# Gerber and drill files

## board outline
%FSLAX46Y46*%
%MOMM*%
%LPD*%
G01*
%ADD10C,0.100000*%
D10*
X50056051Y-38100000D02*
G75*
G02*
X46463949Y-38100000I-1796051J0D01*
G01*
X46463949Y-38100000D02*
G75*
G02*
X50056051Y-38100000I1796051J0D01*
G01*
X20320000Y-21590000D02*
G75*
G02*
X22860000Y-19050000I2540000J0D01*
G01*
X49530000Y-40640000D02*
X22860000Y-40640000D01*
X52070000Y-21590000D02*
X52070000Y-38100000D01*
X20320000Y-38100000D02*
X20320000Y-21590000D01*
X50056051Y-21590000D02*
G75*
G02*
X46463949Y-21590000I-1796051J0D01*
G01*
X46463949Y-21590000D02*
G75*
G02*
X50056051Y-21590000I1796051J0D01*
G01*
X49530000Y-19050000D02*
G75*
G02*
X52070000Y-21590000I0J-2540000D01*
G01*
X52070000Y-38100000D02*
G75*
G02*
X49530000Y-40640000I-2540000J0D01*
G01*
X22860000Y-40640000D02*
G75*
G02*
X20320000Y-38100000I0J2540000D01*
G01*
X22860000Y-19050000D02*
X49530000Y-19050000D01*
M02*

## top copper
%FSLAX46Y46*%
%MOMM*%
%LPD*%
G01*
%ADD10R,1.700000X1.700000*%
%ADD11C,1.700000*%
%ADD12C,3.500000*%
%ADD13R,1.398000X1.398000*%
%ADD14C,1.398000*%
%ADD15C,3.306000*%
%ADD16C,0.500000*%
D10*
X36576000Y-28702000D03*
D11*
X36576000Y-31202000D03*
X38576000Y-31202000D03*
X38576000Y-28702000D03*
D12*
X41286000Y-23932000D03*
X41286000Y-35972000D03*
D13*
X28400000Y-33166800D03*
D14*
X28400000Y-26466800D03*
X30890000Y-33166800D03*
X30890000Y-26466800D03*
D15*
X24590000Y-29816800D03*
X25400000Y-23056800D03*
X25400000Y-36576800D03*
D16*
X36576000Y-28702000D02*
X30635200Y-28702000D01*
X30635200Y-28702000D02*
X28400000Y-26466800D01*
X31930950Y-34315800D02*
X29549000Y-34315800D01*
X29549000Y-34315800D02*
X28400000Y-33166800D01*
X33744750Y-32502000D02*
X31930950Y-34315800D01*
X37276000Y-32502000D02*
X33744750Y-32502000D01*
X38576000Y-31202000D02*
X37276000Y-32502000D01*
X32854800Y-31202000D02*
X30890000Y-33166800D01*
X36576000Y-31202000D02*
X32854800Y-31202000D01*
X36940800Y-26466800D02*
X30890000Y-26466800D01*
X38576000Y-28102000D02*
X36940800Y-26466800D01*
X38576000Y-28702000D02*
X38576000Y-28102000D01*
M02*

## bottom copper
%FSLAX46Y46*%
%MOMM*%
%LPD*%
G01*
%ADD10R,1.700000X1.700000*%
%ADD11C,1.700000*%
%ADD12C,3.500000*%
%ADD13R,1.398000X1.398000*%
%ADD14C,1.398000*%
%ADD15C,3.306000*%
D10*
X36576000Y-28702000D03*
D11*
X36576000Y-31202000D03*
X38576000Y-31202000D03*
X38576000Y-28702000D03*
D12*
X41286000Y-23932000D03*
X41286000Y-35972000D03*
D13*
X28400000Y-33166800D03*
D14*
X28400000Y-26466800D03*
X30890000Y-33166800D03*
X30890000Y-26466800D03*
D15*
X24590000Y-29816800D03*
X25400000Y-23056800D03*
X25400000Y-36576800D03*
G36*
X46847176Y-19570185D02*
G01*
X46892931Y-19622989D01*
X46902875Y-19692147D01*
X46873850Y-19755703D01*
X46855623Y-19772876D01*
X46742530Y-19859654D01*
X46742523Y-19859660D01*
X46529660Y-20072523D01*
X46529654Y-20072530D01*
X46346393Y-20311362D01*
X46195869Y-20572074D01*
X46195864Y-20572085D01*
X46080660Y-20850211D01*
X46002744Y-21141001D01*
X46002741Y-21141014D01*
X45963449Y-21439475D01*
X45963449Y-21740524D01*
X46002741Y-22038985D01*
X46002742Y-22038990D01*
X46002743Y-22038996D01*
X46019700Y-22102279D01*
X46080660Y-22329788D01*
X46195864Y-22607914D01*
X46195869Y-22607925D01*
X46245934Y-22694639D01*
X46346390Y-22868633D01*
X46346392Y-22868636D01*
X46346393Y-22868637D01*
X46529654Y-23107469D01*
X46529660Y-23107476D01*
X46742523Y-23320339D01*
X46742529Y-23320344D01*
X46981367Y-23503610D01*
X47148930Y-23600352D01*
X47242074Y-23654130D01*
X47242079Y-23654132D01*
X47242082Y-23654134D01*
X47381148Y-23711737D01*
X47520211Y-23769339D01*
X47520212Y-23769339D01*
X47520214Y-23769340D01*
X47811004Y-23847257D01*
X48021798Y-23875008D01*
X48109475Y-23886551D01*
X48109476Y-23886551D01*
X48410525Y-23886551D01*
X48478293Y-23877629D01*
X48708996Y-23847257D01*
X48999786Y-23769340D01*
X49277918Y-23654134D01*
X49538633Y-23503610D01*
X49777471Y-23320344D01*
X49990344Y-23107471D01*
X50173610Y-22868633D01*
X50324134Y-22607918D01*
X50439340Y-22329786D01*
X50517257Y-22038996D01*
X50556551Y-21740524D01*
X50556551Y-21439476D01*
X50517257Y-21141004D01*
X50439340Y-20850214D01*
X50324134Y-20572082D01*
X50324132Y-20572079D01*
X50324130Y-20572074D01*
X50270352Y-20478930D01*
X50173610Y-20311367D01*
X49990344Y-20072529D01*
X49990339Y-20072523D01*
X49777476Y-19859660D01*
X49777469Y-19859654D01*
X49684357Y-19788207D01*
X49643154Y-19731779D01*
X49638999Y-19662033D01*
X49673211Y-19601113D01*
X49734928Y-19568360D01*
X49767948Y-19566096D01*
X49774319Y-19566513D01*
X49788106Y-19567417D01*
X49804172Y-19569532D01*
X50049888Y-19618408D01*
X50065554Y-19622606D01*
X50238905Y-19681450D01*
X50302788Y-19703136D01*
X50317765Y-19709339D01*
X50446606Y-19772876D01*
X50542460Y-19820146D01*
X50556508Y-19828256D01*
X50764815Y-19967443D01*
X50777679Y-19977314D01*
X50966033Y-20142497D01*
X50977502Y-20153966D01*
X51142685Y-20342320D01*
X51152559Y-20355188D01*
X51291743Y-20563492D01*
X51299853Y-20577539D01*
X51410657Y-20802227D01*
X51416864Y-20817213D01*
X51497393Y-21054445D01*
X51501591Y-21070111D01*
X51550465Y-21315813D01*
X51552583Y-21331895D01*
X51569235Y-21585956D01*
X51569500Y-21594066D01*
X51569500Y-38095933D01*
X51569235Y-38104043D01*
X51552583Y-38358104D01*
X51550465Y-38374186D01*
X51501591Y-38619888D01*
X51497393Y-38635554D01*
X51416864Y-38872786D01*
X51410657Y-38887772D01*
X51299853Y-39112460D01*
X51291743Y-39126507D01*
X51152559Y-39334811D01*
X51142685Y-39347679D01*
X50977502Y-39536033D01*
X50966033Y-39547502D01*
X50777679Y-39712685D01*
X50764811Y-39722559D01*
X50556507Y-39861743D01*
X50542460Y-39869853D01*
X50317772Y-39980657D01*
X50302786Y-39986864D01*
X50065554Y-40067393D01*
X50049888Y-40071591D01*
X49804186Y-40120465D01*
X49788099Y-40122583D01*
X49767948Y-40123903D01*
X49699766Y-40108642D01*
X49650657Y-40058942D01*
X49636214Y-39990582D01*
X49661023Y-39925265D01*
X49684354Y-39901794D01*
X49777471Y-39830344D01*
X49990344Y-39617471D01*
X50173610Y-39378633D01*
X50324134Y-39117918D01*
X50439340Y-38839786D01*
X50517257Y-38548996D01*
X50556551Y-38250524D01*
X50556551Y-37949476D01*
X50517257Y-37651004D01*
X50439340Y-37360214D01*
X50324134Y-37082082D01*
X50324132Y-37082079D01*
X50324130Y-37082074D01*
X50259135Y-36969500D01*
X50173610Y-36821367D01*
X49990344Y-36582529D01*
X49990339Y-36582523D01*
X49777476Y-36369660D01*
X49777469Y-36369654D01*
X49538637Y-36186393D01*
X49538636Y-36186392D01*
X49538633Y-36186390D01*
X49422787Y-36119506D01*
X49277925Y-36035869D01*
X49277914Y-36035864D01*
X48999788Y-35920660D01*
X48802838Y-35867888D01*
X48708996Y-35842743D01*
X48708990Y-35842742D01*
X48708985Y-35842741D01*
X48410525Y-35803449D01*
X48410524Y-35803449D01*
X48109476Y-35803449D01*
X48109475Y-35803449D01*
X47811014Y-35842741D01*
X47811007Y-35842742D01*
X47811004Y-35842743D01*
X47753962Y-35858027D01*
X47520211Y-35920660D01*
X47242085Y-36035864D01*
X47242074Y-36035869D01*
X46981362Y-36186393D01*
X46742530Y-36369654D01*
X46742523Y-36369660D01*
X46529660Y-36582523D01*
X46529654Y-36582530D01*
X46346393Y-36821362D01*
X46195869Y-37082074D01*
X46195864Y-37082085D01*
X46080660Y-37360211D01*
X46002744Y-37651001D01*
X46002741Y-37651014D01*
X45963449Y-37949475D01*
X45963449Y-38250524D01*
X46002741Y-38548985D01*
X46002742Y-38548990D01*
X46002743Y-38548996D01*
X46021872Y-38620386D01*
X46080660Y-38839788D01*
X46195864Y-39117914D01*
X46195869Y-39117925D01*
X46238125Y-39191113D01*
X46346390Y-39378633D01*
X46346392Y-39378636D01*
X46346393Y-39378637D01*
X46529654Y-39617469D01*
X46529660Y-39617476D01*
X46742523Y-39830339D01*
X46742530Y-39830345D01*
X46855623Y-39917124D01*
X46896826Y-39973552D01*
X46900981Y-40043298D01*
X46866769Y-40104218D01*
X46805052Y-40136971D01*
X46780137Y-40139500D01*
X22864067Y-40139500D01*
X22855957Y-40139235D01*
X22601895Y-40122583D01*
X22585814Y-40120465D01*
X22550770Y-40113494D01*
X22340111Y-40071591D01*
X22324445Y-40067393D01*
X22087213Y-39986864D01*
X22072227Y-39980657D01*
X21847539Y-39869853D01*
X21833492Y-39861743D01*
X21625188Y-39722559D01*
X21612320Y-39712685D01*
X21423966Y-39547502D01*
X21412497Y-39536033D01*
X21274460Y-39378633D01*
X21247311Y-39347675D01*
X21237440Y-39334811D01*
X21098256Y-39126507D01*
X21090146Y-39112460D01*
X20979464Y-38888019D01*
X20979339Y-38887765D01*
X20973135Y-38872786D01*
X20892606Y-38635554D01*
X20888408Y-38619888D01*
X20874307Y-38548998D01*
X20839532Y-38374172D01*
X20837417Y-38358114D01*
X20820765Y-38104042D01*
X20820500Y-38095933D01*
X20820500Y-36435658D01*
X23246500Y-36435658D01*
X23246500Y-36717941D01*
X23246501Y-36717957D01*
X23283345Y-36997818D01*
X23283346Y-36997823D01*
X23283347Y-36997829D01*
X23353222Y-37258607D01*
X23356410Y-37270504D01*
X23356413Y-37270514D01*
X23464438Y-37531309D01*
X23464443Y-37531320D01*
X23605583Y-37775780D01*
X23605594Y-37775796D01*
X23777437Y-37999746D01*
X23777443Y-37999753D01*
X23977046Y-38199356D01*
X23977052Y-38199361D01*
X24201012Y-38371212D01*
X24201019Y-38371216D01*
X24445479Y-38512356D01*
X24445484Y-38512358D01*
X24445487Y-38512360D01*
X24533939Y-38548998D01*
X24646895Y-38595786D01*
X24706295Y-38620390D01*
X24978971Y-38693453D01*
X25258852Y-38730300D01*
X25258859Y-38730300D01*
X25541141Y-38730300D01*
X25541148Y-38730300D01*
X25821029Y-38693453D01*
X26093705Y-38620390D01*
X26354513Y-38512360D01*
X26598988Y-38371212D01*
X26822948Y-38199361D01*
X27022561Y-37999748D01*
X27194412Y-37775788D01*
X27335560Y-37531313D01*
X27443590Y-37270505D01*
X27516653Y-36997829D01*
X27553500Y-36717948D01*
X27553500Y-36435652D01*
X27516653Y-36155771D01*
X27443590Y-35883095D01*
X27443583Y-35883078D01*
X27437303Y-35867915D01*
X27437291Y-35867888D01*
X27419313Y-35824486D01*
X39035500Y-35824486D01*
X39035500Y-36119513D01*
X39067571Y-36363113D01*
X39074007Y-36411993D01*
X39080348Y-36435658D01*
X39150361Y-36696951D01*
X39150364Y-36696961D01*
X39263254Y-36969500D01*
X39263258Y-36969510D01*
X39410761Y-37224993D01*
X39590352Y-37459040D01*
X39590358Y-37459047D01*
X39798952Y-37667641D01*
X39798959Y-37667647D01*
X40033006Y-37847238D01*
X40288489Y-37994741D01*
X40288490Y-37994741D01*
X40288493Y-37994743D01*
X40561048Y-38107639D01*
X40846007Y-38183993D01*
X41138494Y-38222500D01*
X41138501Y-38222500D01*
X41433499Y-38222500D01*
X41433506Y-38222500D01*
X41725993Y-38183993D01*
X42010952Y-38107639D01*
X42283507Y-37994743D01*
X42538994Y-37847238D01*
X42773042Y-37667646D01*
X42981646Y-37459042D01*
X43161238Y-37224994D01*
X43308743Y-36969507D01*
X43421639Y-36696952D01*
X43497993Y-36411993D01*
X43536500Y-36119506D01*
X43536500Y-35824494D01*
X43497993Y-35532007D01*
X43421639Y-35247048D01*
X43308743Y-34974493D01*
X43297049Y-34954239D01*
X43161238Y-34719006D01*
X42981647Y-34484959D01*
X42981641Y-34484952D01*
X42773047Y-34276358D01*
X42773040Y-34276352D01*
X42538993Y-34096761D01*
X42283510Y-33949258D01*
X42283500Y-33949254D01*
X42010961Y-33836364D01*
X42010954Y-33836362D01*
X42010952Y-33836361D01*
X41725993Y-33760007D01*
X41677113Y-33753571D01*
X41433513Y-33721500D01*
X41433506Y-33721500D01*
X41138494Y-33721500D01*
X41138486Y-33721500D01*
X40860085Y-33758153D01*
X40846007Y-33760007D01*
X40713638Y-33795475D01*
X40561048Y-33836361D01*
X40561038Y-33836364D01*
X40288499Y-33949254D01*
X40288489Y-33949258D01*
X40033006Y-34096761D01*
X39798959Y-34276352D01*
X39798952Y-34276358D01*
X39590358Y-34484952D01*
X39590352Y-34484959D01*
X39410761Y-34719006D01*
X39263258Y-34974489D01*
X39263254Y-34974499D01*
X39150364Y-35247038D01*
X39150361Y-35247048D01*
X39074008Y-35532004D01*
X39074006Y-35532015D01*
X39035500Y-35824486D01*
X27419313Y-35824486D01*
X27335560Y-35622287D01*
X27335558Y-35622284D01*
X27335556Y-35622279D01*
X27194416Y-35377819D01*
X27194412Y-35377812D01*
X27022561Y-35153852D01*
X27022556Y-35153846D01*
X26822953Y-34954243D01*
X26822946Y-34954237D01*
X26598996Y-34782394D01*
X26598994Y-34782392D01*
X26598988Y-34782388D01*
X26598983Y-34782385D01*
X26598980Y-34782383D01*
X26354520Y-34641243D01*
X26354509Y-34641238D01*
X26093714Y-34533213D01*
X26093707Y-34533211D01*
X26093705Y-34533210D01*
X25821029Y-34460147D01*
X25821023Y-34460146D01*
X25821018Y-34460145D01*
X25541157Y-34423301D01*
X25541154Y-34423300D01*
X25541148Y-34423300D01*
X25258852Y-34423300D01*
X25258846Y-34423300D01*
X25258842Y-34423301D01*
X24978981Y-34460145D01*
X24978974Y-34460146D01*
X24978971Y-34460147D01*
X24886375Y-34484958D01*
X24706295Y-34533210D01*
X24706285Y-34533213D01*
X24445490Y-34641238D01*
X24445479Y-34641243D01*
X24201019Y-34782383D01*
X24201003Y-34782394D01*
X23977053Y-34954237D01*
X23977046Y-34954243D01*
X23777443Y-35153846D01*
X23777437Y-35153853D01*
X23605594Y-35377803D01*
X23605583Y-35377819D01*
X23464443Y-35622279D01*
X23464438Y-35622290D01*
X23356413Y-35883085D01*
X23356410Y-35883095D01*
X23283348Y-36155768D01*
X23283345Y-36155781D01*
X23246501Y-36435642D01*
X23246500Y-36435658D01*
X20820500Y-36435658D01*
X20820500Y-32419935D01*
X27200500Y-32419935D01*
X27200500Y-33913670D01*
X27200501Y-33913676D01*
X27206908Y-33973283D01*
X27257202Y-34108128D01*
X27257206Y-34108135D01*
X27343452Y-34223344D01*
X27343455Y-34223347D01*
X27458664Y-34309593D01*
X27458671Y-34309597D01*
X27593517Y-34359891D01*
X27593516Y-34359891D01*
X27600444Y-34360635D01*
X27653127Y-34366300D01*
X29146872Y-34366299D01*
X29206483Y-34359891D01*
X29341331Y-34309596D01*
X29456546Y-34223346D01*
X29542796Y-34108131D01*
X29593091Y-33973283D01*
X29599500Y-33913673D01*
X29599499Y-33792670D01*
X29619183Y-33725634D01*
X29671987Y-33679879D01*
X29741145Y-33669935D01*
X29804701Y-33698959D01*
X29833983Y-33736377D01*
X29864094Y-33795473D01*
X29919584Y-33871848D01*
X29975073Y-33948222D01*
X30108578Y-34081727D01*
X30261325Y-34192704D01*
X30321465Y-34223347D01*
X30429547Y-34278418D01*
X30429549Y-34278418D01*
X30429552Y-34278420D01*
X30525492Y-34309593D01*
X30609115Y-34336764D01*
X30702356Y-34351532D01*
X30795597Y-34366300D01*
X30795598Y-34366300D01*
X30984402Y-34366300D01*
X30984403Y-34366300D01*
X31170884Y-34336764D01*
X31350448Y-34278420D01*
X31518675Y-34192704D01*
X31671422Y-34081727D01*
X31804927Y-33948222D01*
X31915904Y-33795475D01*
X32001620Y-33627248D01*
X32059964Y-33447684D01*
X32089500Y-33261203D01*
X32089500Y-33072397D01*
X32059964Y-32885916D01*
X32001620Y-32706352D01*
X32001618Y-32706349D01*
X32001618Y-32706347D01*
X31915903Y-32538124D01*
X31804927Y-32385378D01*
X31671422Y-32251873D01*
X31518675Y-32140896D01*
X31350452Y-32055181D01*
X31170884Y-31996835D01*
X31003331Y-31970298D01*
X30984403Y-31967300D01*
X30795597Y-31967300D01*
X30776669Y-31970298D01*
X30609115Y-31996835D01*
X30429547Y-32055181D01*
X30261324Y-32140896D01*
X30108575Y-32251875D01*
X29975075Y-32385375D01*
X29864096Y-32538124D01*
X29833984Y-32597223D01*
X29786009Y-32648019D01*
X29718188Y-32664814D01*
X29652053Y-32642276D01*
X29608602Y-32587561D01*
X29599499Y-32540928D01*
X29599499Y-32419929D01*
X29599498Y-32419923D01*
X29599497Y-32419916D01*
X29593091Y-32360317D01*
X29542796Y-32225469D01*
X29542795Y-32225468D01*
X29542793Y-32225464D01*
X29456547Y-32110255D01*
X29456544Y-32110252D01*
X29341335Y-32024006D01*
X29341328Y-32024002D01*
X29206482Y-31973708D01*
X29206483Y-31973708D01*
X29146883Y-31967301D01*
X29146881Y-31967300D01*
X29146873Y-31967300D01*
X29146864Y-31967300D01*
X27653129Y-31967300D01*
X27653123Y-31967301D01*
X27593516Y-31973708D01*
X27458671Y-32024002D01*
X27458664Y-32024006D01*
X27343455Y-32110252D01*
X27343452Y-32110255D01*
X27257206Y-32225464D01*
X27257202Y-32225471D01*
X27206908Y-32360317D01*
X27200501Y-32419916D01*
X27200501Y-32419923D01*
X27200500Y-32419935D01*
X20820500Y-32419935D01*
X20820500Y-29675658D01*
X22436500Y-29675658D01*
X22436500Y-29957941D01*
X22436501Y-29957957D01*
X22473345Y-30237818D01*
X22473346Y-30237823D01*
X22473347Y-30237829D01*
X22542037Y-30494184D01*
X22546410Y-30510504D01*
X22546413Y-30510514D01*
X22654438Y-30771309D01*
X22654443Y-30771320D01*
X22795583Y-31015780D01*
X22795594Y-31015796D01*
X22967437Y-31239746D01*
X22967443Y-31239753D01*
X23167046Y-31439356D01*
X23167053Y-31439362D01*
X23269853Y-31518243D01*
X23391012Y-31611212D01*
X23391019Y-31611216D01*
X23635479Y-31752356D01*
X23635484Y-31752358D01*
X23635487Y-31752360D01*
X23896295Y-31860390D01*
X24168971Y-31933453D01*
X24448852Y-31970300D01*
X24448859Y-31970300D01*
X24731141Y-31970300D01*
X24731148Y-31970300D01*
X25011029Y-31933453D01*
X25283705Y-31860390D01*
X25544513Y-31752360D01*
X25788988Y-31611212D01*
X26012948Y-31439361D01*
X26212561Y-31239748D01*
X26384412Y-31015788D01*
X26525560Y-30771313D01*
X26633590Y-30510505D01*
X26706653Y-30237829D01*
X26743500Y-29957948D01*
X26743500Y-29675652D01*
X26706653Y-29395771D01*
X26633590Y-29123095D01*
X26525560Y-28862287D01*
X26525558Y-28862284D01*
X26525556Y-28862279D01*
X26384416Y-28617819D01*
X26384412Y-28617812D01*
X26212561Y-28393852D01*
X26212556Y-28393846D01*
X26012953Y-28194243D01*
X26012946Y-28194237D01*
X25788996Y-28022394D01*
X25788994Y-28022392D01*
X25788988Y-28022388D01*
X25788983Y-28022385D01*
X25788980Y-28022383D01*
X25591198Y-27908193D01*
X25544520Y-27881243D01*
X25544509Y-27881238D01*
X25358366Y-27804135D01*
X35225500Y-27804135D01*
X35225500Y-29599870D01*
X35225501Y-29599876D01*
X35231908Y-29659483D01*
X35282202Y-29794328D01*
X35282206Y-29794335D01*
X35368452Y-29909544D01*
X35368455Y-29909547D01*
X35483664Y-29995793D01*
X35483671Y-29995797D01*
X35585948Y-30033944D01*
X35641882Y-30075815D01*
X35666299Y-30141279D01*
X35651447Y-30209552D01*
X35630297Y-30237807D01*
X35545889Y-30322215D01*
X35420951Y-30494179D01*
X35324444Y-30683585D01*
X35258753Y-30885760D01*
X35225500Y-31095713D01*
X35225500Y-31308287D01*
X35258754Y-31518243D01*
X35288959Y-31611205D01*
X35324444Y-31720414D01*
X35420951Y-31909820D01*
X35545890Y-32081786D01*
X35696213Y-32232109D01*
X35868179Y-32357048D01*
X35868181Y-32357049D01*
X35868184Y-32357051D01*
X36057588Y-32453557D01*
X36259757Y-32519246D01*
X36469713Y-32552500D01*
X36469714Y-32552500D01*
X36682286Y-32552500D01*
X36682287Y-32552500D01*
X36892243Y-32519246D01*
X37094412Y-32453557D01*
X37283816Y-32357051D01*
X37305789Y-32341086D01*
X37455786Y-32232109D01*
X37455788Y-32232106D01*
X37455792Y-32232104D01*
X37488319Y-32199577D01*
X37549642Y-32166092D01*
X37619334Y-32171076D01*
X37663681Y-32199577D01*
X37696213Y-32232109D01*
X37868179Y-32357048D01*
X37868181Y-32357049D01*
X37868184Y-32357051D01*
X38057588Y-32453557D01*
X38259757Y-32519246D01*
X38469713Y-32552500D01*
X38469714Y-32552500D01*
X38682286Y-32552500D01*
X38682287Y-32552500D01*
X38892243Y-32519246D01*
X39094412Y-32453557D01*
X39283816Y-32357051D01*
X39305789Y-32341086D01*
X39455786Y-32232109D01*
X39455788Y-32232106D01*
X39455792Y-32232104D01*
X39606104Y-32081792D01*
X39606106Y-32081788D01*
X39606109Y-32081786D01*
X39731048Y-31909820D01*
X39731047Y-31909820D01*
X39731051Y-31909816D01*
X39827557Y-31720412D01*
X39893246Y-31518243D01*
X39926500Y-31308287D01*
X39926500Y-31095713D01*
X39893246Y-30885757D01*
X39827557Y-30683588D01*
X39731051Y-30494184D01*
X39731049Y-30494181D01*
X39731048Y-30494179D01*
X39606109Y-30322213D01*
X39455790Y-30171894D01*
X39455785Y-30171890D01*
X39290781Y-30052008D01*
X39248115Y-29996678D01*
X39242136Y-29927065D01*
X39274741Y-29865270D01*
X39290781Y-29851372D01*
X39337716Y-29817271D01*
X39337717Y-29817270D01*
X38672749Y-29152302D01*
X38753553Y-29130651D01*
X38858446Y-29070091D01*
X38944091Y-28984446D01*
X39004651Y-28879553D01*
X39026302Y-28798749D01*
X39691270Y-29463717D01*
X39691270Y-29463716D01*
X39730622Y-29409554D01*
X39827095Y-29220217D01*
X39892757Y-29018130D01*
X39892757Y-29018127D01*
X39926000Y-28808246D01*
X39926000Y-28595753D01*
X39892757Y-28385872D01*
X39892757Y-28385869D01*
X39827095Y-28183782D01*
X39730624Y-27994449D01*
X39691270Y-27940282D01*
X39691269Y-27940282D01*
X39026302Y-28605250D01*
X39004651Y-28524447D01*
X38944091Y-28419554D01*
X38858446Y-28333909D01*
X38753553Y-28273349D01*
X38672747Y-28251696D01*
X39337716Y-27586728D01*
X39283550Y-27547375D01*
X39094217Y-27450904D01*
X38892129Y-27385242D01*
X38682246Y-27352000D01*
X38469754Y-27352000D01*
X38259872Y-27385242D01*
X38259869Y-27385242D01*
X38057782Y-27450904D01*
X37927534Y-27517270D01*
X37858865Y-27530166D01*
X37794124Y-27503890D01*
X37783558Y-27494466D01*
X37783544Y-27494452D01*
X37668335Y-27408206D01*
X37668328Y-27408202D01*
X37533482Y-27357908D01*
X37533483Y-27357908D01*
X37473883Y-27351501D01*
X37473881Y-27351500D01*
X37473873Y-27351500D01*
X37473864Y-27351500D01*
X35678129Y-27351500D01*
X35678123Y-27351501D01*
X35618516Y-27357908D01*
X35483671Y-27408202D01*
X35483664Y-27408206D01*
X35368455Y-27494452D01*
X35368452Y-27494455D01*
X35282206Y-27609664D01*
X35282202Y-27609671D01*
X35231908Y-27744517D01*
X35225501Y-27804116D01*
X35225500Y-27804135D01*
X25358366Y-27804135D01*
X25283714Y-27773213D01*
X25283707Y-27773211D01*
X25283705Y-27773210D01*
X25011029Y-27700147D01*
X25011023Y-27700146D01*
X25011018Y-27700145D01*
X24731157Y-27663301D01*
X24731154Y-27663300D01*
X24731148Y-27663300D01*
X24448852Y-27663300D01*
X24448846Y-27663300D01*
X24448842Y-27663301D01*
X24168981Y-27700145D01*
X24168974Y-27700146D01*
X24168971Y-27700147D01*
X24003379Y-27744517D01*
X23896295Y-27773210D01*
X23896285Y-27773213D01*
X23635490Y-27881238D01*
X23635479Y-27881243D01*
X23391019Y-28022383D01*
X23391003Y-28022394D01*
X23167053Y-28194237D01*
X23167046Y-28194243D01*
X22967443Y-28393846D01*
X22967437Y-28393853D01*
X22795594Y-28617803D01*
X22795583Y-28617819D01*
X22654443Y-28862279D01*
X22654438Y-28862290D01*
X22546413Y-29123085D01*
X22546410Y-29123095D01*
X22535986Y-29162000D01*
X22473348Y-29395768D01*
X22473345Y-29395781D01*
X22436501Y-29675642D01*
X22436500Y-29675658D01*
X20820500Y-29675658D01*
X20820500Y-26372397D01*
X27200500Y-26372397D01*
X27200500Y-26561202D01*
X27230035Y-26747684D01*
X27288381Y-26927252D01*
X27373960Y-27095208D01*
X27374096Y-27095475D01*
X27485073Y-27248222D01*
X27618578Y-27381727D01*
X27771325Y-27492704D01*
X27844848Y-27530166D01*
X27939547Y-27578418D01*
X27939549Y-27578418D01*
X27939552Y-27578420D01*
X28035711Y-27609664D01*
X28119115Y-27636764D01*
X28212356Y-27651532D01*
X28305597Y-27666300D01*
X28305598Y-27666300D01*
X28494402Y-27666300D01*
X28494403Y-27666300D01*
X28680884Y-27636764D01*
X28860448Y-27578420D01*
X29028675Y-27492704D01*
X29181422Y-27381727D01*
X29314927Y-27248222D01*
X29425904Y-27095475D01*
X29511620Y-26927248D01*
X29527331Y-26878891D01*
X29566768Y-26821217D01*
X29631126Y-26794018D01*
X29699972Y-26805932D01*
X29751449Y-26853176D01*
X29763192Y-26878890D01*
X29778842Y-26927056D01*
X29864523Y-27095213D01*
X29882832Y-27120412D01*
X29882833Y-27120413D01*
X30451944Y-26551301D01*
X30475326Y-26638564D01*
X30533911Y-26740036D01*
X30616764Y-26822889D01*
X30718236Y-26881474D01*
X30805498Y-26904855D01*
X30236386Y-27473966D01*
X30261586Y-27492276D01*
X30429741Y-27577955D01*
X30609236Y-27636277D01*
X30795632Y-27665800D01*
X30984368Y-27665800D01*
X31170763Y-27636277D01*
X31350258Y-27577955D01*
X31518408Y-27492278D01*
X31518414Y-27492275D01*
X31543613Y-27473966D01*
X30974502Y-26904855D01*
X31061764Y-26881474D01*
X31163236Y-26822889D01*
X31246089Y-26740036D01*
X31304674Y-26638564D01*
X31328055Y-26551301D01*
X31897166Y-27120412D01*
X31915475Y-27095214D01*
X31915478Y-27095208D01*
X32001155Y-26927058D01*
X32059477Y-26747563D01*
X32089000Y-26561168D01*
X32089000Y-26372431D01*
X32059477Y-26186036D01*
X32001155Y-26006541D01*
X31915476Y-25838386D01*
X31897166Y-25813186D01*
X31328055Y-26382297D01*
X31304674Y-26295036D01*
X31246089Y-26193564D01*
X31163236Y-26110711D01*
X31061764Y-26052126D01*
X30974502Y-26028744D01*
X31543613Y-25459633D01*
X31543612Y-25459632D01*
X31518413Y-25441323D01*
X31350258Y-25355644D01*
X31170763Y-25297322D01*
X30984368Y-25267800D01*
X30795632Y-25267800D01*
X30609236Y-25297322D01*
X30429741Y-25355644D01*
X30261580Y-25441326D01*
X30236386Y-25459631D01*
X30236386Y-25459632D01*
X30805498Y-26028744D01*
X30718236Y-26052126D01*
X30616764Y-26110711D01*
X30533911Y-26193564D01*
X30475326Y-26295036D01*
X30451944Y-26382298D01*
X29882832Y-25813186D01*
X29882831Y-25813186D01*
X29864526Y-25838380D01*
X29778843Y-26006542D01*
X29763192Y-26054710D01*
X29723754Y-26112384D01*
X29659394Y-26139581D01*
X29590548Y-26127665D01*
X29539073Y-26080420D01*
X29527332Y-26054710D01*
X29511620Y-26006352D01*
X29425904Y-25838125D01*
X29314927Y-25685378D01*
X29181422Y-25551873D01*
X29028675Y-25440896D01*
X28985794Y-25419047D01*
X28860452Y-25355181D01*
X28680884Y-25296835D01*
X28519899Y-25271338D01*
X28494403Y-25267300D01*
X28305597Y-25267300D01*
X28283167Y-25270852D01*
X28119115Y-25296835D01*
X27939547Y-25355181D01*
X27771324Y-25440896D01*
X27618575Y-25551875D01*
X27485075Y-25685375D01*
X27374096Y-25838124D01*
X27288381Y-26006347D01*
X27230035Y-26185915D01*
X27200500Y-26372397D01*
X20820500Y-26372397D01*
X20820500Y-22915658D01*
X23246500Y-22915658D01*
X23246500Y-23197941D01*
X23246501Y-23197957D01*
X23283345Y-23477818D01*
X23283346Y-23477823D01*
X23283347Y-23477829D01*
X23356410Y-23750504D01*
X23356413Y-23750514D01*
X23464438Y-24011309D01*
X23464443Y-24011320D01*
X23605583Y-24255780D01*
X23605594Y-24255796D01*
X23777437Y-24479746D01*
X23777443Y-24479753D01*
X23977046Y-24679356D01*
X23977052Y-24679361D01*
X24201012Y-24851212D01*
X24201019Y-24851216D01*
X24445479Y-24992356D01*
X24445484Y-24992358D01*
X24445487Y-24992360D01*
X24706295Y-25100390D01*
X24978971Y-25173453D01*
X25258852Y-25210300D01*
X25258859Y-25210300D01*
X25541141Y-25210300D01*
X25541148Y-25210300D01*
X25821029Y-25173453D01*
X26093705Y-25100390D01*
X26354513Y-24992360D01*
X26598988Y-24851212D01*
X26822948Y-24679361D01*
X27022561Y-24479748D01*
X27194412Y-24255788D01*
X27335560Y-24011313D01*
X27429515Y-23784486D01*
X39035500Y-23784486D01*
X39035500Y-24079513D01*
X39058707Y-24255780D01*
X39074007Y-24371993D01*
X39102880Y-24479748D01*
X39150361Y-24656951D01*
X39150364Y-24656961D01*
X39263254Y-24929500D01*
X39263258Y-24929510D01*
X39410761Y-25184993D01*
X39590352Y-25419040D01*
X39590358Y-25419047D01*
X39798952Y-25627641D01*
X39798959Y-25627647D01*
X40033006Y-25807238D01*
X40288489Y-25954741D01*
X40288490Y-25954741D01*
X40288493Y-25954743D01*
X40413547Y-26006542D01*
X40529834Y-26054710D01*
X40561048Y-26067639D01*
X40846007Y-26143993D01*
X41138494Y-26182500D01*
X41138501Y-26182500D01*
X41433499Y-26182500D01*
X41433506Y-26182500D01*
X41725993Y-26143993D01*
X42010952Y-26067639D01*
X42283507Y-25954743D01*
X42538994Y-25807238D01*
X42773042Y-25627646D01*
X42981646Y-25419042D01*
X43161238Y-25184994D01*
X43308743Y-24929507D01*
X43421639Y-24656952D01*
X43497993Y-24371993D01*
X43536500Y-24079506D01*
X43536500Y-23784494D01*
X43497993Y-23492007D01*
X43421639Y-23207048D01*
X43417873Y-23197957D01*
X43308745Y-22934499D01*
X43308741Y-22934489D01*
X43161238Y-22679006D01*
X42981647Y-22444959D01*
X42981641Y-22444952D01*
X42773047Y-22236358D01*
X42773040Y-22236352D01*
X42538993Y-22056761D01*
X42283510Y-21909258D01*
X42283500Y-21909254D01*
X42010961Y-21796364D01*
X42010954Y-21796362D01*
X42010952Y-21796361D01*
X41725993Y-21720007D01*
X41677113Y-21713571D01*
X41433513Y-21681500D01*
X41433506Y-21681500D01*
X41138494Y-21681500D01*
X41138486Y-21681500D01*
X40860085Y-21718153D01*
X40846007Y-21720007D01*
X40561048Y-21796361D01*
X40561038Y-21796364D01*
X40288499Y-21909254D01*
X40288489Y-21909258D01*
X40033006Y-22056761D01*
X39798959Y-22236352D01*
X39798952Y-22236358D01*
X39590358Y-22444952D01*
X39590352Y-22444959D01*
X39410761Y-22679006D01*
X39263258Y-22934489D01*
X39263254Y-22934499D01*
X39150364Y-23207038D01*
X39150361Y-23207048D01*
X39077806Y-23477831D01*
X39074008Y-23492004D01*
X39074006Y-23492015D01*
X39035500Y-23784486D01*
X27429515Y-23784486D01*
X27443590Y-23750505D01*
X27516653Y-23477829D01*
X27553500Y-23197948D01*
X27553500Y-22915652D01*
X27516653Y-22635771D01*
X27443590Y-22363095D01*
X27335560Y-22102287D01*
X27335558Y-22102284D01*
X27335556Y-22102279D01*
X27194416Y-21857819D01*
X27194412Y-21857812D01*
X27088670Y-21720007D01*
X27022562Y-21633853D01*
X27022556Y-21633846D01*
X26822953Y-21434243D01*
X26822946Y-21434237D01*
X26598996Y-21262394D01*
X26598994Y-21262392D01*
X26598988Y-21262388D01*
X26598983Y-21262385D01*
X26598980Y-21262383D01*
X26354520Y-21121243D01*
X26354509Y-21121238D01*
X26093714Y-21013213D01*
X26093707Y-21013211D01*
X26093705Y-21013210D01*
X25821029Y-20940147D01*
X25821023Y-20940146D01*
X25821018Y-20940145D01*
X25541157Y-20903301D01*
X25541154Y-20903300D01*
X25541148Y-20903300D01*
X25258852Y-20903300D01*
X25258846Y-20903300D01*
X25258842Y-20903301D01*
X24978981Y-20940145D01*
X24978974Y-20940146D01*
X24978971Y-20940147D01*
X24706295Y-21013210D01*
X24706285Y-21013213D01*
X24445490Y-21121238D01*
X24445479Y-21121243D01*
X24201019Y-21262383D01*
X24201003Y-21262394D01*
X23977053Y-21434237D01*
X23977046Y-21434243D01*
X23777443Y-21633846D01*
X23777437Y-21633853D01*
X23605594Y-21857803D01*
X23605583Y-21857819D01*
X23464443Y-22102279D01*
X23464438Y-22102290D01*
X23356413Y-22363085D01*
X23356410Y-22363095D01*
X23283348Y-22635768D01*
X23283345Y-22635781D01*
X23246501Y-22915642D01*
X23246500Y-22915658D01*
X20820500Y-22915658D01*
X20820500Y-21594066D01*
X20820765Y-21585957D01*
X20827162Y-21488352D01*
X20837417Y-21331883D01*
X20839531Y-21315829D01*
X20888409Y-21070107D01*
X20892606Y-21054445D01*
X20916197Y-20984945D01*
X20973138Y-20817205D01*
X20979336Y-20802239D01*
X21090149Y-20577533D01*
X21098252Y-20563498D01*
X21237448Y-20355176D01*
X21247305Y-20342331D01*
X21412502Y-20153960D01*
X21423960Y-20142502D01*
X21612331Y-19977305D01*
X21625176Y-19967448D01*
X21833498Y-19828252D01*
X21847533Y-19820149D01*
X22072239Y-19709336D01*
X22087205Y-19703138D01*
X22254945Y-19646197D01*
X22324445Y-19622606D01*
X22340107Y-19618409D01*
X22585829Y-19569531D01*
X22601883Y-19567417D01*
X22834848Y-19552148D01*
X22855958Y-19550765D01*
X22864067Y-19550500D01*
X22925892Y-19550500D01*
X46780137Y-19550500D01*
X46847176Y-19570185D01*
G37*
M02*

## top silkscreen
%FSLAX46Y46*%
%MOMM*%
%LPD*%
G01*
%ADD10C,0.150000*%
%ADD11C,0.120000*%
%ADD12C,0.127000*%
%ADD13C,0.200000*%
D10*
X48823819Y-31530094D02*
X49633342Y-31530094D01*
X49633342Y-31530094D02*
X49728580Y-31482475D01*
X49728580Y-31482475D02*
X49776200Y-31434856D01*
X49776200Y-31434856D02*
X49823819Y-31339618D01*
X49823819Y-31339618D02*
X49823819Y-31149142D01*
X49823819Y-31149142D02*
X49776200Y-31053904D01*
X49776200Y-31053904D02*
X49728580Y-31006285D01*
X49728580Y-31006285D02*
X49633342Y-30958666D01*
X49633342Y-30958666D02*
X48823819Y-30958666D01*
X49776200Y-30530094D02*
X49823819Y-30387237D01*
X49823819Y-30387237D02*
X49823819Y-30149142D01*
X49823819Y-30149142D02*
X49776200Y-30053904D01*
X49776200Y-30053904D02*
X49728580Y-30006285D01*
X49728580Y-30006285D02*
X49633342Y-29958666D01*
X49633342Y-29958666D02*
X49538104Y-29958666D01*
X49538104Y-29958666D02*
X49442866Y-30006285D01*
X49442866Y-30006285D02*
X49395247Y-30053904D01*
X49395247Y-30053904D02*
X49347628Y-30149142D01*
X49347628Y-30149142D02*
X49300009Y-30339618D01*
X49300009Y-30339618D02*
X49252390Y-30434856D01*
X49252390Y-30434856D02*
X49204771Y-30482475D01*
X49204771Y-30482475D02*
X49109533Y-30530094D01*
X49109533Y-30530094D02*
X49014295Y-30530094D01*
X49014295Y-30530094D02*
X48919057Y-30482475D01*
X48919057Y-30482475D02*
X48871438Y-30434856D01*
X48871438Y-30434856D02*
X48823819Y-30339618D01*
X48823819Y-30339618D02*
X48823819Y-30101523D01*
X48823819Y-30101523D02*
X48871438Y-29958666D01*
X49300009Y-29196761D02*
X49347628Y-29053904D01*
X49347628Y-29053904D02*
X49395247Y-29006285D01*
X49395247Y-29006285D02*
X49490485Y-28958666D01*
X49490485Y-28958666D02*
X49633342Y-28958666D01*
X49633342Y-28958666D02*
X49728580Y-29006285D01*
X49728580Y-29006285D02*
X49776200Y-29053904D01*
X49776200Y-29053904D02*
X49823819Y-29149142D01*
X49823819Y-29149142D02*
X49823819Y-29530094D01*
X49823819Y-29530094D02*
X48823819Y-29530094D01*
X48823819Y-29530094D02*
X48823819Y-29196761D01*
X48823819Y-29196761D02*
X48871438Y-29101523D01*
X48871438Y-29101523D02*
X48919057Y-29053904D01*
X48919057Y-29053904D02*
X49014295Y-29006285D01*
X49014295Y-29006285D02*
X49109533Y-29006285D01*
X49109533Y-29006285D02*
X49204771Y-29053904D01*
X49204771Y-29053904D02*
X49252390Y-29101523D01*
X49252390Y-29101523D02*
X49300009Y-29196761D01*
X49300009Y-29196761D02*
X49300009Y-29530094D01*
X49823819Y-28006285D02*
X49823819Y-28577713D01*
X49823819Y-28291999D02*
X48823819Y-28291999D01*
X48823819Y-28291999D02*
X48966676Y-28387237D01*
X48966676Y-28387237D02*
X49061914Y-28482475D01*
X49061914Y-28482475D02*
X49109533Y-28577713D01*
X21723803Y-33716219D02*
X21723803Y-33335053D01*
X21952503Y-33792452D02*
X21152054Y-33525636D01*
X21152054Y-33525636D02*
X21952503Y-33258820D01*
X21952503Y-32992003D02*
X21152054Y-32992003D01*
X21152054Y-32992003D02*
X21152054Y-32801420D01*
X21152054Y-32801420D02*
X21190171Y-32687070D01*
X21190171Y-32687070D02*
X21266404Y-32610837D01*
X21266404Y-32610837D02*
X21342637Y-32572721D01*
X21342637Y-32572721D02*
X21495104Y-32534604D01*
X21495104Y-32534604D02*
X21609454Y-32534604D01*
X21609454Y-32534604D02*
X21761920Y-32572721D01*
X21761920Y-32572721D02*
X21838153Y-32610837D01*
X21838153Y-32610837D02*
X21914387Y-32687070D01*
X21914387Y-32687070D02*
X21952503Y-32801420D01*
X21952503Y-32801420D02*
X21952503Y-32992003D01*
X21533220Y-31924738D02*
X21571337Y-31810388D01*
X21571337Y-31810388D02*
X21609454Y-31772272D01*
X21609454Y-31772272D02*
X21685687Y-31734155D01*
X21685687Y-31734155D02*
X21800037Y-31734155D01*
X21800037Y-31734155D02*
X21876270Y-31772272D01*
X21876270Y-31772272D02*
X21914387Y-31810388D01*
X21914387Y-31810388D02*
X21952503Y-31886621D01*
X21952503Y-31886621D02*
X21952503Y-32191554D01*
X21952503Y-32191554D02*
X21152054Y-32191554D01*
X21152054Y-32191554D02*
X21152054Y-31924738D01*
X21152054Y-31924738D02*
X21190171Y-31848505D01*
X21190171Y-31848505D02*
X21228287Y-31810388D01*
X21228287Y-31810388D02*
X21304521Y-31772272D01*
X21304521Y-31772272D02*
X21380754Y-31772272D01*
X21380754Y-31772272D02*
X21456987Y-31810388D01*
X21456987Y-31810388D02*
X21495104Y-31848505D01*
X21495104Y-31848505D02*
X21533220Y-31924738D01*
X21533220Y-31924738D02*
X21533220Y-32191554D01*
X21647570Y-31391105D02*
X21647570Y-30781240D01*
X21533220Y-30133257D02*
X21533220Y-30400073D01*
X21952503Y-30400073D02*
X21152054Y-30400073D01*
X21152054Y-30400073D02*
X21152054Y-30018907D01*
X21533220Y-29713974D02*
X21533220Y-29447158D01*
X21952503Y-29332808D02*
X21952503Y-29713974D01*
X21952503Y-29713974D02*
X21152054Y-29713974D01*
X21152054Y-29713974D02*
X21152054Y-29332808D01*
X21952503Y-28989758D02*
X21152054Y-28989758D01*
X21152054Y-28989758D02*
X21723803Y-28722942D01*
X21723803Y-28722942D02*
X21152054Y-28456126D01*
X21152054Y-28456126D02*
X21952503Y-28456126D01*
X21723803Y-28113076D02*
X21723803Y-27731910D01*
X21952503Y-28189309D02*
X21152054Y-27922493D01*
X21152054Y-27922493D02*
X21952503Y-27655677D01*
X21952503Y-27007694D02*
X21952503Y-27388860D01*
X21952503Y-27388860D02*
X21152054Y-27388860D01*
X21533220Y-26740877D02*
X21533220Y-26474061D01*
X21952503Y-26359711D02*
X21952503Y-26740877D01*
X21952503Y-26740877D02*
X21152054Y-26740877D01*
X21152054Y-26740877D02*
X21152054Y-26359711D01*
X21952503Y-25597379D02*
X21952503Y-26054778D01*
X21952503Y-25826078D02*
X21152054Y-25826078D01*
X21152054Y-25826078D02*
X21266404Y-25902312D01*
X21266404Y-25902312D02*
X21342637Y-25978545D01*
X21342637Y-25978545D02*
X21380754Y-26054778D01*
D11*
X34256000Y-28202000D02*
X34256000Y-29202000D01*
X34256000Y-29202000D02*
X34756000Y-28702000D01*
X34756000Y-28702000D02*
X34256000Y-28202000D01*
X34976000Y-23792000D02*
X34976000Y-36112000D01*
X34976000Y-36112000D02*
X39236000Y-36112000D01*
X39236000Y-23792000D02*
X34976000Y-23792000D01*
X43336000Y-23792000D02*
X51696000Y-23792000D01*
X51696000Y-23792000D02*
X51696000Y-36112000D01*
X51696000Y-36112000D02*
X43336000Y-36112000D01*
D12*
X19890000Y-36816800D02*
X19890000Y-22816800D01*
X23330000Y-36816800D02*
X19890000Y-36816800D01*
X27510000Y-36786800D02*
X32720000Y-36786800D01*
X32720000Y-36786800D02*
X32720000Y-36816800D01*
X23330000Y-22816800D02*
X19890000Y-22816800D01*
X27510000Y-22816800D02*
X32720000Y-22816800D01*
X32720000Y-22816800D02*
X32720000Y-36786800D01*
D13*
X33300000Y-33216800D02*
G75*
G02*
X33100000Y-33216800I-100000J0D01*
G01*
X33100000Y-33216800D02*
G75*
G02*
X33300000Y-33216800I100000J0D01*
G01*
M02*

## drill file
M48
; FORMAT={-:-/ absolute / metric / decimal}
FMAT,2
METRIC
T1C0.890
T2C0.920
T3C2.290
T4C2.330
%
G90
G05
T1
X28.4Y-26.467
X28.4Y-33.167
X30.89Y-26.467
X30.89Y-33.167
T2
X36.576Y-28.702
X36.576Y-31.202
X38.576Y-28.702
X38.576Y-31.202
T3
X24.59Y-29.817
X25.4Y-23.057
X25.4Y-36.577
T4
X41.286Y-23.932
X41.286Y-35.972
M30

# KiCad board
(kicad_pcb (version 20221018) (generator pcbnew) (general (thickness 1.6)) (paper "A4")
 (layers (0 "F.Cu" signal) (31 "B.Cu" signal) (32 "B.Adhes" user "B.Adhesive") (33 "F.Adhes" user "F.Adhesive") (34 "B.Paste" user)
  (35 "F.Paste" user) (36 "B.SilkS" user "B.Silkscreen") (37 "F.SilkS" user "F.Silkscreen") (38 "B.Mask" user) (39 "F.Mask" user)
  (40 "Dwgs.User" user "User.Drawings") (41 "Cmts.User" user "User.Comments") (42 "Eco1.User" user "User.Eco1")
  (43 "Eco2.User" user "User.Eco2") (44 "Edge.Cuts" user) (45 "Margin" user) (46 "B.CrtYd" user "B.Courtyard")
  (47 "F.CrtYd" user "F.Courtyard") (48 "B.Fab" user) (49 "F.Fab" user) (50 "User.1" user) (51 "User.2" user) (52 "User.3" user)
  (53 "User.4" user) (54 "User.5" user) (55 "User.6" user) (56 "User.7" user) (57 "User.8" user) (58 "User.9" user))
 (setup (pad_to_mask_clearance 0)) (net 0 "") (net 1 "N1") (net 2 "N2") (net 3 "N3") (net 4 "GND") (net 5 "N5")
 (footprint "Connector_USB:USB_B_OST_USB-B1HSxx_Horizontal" (layer "F.Cu") (at 36.576 28.702)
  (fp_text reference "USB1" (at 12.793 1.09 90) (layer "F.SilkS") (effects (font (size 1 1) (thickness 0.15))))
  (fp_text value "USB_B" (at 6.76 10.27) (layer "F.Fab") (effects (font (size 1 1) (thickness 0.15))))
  (fp_line (start -2.32 -0.5) (end -2.32 0.5) (stroke (width 0.12) (type solid)) (layer "F.SilkS"))
  (fp_line (start -2.32 0.5) (end -1.82 0) (stroke (width 0.12) (type solid)) (layer "F.SilkS"))
  (fp_line (start -1.82 0) (end -2.32 -0.5) (stroke (width 0.12) (type solid)) (layer "F.SilkS"))
  (fp_line (start -1.6 -4.91) (end -1.6 7.41) (stroke (width 0.12) (type solid)) (layer "F.SilkS"))
  (fp_line (start -1.6 7.41) (end 2.66 7.41) (stroke (width 0.12) (type solid)) (layer "F.SilkS"))
  (fp_line (start 2.66 -4.91) (end -1.6 -4.91) (stroke (width 0.12) (type solid)) (layer "F.SilkS"))
  (fp_line (start 6.76 -4.91) (end 15.12 -4.91) (stroke (width 0.12) (type solid)) (layer "F.SilkS"))
  (fp_line (start 15.12 -4.91) (end 15.12 7.41) (stroke (width 0.12) (type solid)) (layer "F.SilkS"))
  (fp_line (start 15.12 7.41) (end 6.76 7.41) (stroke (width 0.12) (type solid)) (layer "F.SilkS"))
  (pad "1" thru_hole rect (at 0 0) (size 1.7 1.7) (drill 0.92) (layers "*.Cu" "*.Mask") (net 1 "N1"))
  (pad "2" thru_hole circle (at 0 2.5) (size 1.7 1.7) (drill 0.92) (layers "*.Cu" "*.Mask") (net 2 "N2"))
  (pad "3" thru_hole circle (at 2 2.5) (size 1.7 1.7) (drill 0.92) (layers "*.Cu" "*.Mask") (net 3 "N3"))
  (pad "4" thru_hole circle (at 2 0) (size 1.7 1.7) (drill 0.92) (layers "*.Cu" "*.Mask") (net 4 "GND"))
  (pad "5" thru_hole circle (at 4.71 -4.77) (size 3.5 3.5) (drill 2.33) (layers "*.Cu" "*.Mask") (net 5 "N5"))
  (pad "5" thru_hole circle (at 4.71 7.27) (size 3.5 3.5) (drill 2.33) (layers "*.Cu" "*.Mask") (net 5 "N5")))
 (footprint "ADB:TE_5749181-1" (layer "F.Cu") (at 28.4 29.8168 90)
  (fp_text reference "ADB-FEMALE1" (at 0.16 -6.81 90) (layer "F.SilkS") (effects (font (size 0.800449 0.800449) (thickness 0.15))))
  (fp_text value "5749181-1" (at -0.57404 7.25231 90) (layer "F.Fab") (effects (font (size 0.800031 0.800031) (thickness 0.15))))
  (fp_line (start -7 -8.51) (end 7 -8.51) (stroke (width 0.127) (type solid)) (layer "F.SilkS"))
  (fp_line (start -7 -5.07) (end -7 -8.51) (stroke (width 0.127) (type solid)) (layer "F.SilkS"))
  (fp_line (start -6.97 -0.89) (end -6.97 4.32) (stroke (width 0.127) (type solid)) (layer "F.SilkS"))
  (fp_line (start -6.97 4.32) (end -7 4.32) (stroke (width 0.127) (type solid)) (layer "F.SilkS"))
  (fp_line (start 7 -5.07) (end 7 -8.51) (stroke (width 0.127) (type solid)) (layer "F.SilkS"))
  (fp_line (start 7 -0.89) (end 7 4.32) (stroke (width 0.127) (type solid)) (layer "F.SilkS"))
  (fp_line (start 7 4.32) (end -6.97 4.32) (stroke (width 0.127) (type solid)) (layer "F.SilkS"))
  (fp_circle (center -3.4 4.8) (end -3.3 4.8) (stroke (width 0.2) (type solid)) (fill none) (layer "F.SilkS"))
  (pad "1" thru_hole rect (at -3.35 0 90) (size 1.398 1.398) (drill 0.89) (layers "*.Cu" "*.Mask") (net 3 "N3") (solder_mask_margin 0.102))
  (pad "2" thru_hole circle (at 3.35 0 90) (size 1.398 1.398) (drill 0.89) (layers "*.Cu" "*.Mask") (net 1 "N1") (solder_mask_margin 0.102))
  (pad "3" thru_hole circle (at -3.35 2.49 90) (size 1.398 1.398) (drill 0.89) (layers "*.Cu" "*.Mask") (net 2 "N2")
   (solder_mask_margin 0.102))
  (pad "4" thru_hole circle (at 3.35 2.49 90) (size 1.398 1.398) (drill 0.89) (layers "*.Cu" "*.Mask") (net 4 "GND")
   (solder_mask_margin 0.102))
  (pad "5" thru_hole circle (at 0 -3.81 90) (size 3.306 3.306) (drill 2.29) (layers "*.Cu" "*.Mask") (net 5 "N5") (solder_mask_margin 0.102))
  (pad "6" thru_hole circle (at 6.76 -3 90) (size 3.306 3.306) (drill 2.29) (layers "*.Cu" "*.Mask") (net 5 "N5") (solder_mask_margin 0.102))
  (pad "7" thru_hole circle (at -6.76 -3 90) (size 3.306 3.306) (drill 2.29) (layers "*.Cu" "*.Mask") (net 5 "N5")
   (solder_mask_margin 0.102)))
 (gr_circle (center 48.26 38.1) (end 49.53 39.37) (stroke (width 0.1) (type default)) (fill none) (layer "Edge.Cuts"))
 (gr_arc (start 20.32 21.59) (mid 21.063949 19.793949) (end 22.86 19.05) (stroke (width 0.1) (type default)) (layer "Edge.Cuts"))
 (gr_line (start 49.53 40.64) (end 22.86 40.64) (stroke (width 0.1) (type default)) (layer "Edge.Cuts"))
 (gr_line (start 52.07 21.59) (end 52.07 38.1) (stroke (width 0.1) (type default)) (layer "Edge.Cuts"))
 (gr_line (start 20.32 38.1) (end 20.32 21.59) (stroke (width 0.1) (type default)) (layer "Edge.Cuts"))
 (gr_circle (center 48.26 21.59) (end 49.53 22.86) (stroke (width 0.1) (type default)) (fill none) (layer "Edge.Cuts"))
 (gr_arc (start 49.53 19.05) (mid 51.326051 19.793949) (end 52.07 21.59) (stroke (width 0.1) (type default)) (layer "Edge.Cuts"))
 (gr_arc (start 52.07 38.1) (mid 51.326051 39.896051) (end 49.53 40.64) (stroke (width 0.1) (type default)) (layer "Edge.Cuts"))
 (gr_arc (start 22.86 40.64) (mid 21.063949 39.896051) (end 20.32 38.1) (stroke (width 0.1) (type default)) (layer "Edge.Cuts"))
 (gr_line (start 22.86 19.05) (end 49.53 19.05) (stroke (width 0.1) (type default)) (layer "Edge.Cuts"))
 (segment (start 36.576 28.702) (end 30.6352 28.702) (width 0.5) (layer "F.Cu") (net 1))
 (segment (start 30.6352 28.702) (end 28.4 26.4668) (width 0.5) (layer "F.Cu") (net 1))
 (segment (start 31.93095 34.3158) (end 29.549 34.3158) (width 0.5) (layer "F.Cu") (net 3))
 (segment (start 29.549 34.3158) (end 28.4 33.1668) (width 0.5) (layer "F.Cu") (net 3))
 (segment (start 33.74475 32.502) (end 31.93095 34.3158) (width 0.5) (layer "F.Cu") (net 3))
 (segment (start 37.276 32.502) (end 33.74475 32.502) (width 0.5) (layer "F.Cu") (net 3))
 (segment (start 38.576 31.202) (end 37.276 32.502) (width 0.5) (layer "F.Cu") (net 3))
 (segment (start 32.8548 31.202) (end 30.89 33.1668) (width 0.5) (layer "F.Cu") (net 2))
 (segment (start 36.576 31.202) (end 32.8548 31.202) (width 0.5) (layer "F.Cu") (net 2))
 (segment (start 36.9408 26.4668) (end 30.89 26.4668) (width 0.5) (layer "F.Cu") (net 4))
 (segment (start 38.576 28.102) (end 36.9408 26.4668) (width 0.5) (layer "F.Cu") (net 4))
 (segment (start 38.576 28.702) (end 38.576 28.102) (width 0.5) (layer "F.Cu") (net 4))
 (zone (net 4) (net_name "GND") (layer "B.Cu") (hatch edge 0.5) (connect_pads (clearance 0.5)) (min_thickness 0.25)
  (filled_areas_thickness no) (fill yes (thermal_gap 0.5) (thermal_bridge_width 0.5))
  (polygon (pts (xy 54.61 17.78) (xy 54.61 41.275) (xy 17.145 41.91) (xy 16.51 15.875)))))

